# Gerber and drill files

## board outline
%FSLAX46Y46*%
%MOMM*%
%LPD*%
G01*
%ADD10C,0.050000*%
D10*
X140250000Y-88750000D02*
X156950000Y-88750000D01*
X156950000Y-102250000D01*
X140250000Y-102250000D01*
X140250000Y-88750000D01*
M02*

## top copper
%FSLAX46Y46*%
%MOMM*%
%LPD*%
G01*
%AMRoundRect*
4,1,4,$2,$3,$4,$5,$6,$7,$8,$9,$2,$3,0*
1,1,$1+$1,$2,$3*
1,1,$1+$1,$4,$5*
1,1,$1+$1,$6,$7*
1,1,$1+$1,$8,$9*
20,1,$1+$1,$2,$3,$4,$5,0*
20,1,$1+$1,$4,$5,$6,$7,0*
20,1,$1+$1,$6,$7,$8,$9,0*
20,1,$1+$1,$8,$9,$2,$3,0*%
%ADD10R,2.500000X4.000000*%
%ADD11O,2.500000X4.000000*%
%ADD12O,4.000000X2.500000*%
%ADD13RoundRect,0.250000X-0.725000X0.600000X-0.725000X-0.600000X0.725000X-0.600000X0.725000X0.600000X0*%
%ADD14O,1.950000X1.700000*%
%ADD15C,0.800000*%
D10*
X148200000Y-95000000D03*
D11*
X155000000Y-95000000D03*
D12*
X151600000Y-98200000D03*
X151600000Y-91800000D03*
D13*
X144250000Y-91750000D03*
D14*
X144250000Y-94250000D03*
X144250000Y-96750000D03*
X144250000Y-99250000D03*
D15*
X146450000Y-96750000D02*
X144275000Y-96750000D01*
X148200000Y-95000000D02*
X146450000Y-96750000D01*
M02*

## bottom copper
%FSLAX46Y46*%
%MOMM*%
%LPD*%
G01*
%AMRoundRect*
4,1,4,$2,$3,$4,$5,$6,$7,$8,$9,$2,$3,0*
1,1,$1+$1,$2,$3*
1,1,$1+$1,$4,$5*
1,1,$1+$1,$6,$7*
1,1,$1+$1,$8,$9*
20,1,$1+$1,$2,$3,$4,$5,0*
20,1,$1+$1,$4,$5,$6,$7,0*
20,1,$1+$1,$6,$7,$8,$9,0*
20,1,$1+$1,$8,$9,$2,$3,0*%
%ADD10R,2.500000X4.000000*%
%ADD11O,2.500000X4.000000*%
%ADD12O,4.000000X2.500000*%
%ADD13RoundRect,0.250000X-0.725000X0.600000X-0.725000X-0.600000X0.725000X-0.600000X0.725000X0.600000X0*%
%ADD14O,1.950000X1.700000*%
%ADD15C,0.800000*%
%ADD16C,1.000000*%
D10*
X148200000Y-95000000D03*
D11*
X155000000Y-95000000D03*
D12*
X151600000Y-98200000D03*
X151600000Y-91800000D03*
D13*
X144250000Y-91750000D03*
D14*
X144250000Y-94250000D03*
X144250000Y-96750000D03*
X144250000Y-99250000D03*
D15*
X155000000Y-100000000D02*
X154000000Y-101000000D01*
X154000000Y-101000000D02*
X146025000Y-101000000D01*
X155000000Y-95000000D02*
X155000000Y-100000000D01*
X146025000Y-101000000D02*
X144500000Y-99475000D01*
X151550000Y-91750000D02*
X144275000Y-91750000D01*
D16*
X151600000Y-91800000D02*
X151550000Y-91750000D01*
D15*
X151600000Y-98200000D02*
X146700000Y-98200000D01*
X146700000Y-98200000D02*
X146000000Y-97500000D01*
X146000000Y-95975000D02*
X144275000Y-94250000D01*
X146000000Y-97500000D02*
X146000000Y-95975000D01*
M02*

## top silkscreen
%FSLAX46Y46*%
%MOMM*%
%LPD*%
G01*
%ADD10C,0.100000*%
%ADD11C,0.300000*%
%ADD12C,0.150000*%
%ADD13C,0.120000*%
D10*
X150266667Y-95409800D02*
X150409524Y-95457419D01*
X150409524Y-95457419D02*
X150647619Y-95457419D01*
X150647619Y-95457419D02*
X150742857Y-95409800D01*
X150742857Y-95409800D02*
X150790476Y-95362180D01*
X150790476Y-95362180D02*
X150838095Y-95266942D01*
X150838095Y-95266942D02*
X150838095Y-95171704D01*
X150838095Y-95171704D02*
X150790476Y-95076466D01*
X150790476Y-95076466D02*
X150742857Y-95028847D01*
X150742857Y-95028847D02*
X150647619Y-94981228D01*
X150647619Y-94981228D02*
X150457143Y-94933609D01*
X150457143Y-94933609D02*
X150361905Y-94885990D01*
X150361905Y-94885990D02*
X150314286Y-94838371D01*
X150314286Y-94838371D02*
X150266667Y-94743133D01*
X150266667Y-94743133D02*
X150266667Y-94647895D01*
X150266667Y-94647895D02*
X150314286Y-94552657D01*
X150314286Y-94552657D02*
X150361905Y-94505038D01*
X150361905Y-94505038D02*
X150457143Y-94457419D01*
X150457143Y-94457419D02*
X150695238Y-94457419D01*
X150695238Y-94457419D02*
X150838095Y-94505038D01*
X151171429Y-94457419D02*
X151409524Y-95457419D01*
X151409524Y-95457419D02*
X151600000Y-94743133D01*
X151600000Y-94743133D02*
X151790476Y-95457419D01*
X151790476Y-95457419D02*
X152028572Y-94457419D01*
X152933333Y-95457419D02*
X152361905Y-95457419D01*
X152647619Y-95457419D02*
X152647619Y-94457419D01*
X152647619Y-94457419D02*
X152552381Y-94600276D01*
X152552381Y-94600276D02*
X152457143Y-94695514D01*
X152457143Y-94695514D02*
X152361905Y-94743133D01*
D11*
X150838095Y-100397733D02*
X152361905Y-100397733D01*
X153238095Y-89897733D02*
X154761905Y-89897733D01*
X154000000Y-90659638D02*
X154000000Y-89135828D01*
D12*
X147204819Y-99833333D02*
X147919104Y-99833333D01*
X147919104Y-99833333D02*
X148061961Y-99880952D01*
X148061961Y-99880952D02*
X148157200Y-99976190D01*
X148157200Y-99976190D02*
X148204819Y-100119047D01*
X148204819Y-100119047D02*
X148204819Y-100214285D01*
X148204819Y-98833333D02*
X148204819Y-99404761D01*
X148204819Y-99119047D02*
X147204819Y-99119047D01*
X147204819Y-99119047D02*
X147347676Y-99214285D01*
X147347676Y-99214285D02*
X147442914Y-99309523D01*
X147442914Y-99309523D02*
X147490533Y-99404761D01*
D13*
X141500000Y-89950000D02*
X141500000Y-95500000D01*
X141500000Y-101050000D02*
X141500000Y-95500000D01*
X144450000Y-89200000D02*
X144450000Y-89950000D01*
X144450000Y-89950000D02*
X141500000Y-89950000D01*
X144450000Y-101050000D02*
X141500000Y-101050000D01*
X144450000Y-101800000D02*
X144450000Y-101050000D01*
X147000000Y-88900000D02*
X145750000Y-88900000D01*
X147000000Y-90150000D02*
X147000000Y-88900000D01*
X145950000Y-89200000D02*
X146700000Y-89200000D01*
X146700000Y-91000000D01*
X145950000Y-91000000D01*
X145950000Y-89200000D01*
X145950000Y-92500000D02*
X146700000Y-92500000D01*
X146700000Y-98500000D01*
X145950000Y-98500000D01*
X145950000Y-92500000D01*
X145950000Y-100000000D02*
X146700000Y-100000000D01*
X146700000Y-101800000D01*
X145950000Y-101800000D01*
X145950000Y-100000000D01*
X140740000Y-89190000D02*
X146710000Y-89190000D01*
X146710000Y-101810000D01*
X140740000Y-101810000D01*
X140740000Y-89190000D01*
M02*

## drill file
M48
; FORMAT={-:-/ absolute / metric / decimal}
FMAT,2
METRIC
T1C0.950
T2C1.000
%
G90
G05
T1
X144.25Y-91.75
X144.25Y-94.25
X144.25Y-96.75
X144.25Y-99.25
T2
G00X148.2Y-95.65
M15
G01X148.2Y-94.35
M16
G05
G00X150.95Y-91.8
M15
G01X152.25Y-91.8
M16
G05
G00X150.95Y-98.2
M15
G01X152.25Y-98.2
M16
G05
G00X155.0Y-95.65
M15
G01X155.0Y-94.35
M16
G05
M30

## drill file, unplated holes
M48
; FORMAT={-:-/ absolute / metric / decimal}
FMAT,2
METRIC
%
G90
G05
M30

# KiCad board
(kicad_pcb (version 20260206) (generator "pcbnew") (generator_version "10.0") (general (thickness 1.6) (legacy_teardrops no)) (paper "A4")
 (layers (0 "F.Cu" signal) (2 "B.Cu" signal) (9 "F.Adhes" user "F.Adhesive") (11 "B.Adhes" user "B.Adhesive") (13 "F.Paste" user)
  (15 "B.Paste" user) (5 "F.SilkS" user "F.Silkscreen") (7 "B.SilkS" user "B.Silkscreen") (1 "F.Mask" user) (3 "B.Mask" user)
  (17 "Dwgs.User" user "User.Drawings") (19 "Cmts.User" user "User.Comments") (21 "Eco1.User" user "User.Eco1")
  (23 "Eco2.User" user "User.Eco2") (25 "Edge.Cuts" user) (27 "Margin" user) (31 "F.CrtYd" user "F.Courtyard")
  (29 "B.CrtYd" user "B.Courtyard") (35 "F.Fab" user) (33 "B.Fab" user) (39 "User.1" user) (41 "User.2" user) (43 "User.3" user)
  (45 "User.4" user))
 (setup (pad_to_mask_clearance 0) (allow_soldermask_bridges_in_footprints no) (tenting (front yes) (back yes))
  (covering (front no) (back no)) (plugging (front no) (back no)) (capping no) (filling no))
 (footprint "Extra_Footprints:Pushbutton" (layer "F.Cu") (at 151.6 95)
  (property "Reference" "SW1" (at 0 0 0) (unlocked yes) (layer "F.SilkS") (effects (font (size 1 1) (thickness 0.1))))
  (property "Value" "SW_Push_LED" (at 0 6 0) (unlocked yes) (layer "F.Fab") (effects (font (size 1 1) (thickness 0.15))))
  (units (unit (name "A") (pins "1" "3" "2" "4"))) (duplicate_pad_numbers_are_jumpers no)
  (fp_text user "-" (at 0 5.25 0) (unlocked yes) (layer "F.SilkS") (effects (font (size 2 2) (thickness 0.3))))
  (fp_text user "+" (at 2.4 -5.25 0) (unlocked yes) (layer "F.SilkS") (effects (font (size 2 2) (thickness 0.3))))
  (pad "1" thru_hole rect (at -3.4 0 90) (size 4 2.5) (drill oval 2.3 1) (layers "*.Cu" "*.Mask") (remove_unused_layers no) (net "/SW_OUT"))
  (pad "2" thru_hole oval (at 3.4 0 90) (size 4 2.5) (drill oval 2.3 1) (layers "*.Cu" "*.Mask") (remove_unused_layers no) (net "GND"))
  (pad "3" thru_hole oval (at 0 3.2) (size 4 2.5) (drill oval 2.3 1) (layers "*.Cu" "*.Mask") (remove_unused_layers no) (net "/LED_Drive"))
  (pad "4" thru_hole oval (at 0 -3.2) (size 4 2.5) (drill oval 2.3 1) (layers "*.Cu" "*.Mask") (remove_unused_layers no) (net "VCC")))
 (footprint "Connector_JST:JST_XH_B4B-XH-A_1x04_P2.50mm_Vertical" (layer "F.Cu") (at 144.25 91.75 -90)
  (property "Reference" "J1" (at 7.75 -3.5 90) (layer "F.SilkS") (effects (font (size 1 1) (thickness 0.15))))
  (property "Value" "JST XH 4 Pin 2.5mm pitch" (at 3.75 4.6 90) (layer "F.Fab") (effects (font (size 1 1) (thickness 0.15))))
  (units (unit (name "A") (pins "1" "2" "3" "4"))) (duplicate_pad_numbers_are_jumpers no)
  (fp_line (start -1.8 2.75) (end 3.75 2.75) (stroke (width 0.12) (type solid)) (layer "F.SilkS"))
  (fp_line (start 9.3 2.75) (end 3.75 2.75) (stroke (width 0.12) (type solid)) (layer "F.SilkS"))
  (fp_line (start -2.55 -0.2) (end -1.8 -0.2) (stroke (width 0.12) (type solid)) (layer "F.SilkS"))
  (fp_line (start -1.8 -0.2) (end -1.8 2.75) (stroke (width 0.12) (type solid)) (layer "F.SilkS"))
  (fp_line (start 9.3 -0.2) (end 9.3 2.75) (stroke (width 0.12) (type solid)) (layer "F.SilkS"))
  (fp_line (start 10.05 -0.2) (end 9.3 -0.2) (stroke (width 0.12) (type solid)) (layer "F.SilkS"))
  (fp_line (start -2.85 -2.75) (end -2.85 -1.5) (stroke (width 0.12) (type solid)) (layer "F.SilkS"))
  (fp_line (start -1.6 -2.75) (end -2.85 -2.75) (stroke (width 0.12) (type solid)) (layer "F.SilkS"))
  (fp_rect (start -2.55 -2.45) (end -0.75 -1.7) (stroke (width 0.12) (type solid)) (fill no) (layer "F.SilkS"))
  (fp_rect (start 0.75 -2.45) (end 6.75 -1.7) (stroke (width 0.12) (type solid)) (fill no) (layer "F.SilkS"))
  (fp_rect (start 8.25 -2.45) (end 10.05 -1.7) (stroke (width 0.12) (type solid)) (fill no) (layer "F.SilkS"))
  (fp_rect (start -2.56 -2.46) (end 10.06 3.51) (stroke (width 0.12) (type solid)) (fill no) (layer "F.SilkS"))
  (pad "1" thru_hole roundrect (at 0 0 270) (size 1.7 1.95) (drill 0.95) (layers "*.Cu" "*.Mask") (remove_unused_layers no)
   (roundrect_rratio 0.147059) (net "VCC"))
  (pad "2" thru_hole oval (at 2.5 0 270) (size 1.7 1.95) (drill 0.95) (layers "*.Cu" "*.Mask") (remove_unused_layers no) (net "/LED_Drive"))
  (pad "3" thru_hole oval (at 5 0 270) (size 1.7 1.95) (drill 0.95) (layers "*.Cu" "*.Mask") (remove_unused_layers no) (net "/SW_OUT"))
  (pad "4" thru_hole oval (at 7.5 0 270) (size 1.7 1.95) (drill 0.95) (layers "*.Cu" "*.Mask") (remove_unused_layers no) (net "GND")))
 (gr_rect (start 140.25 88.75) (end 156.95 102.25) (stroke (width 0.05) (type default)) (fill no) (layer "Edge.Cuts"))
 (segment (start 146.45 96.75) (end 144.275 96.75) (width 0.8) (layer "F.Cu") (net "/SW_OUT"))
 (segment (start 148.2 95) (end 146.45 96.75) (width 0.8) (layer "F.Cu") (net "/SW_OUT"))
 (segment (start 155 100) (end 154 101) (width 0.8) (layer "B.Cu") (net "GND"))
 (segment (start 154 101) (end 146.025 101) (width 0.8) (layer "B.Cu") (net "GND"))
 (segment (start 155 95) (end 155 100) (width 0.8) (layer "B.Cu") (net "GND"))
 (segment (start 146.025 101) (end 144.5 99.475) (width 0.8) (layer "B.Cu") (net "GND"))
 (segment (start 151.6 98.2) (end 146.7 98.2) (width 0.8) (layer "B.Cu") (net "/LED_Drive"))
 (segment (start 146.7 98.2) (end 146 97.5) (width 0.8) (layer "B.Cu") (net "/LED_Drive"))
 (segment (start 146 95.975) (end 144.275 94.25) (width 0.8) (layer "B.Cu") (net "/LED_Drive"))
 (segment (start 146 97.5) (end 146 95.975) (width 0.8) (layer "B.Cu") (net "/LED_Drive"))
 (segment (start 151.55 91.75) (end 144.275 91.75) (width 0.8) (layer "B.Cu") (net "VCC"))
 (segment (start 151.6 91.8) (end 151.55 91.75) (width 1) (layer "B.Cu") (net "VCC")))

